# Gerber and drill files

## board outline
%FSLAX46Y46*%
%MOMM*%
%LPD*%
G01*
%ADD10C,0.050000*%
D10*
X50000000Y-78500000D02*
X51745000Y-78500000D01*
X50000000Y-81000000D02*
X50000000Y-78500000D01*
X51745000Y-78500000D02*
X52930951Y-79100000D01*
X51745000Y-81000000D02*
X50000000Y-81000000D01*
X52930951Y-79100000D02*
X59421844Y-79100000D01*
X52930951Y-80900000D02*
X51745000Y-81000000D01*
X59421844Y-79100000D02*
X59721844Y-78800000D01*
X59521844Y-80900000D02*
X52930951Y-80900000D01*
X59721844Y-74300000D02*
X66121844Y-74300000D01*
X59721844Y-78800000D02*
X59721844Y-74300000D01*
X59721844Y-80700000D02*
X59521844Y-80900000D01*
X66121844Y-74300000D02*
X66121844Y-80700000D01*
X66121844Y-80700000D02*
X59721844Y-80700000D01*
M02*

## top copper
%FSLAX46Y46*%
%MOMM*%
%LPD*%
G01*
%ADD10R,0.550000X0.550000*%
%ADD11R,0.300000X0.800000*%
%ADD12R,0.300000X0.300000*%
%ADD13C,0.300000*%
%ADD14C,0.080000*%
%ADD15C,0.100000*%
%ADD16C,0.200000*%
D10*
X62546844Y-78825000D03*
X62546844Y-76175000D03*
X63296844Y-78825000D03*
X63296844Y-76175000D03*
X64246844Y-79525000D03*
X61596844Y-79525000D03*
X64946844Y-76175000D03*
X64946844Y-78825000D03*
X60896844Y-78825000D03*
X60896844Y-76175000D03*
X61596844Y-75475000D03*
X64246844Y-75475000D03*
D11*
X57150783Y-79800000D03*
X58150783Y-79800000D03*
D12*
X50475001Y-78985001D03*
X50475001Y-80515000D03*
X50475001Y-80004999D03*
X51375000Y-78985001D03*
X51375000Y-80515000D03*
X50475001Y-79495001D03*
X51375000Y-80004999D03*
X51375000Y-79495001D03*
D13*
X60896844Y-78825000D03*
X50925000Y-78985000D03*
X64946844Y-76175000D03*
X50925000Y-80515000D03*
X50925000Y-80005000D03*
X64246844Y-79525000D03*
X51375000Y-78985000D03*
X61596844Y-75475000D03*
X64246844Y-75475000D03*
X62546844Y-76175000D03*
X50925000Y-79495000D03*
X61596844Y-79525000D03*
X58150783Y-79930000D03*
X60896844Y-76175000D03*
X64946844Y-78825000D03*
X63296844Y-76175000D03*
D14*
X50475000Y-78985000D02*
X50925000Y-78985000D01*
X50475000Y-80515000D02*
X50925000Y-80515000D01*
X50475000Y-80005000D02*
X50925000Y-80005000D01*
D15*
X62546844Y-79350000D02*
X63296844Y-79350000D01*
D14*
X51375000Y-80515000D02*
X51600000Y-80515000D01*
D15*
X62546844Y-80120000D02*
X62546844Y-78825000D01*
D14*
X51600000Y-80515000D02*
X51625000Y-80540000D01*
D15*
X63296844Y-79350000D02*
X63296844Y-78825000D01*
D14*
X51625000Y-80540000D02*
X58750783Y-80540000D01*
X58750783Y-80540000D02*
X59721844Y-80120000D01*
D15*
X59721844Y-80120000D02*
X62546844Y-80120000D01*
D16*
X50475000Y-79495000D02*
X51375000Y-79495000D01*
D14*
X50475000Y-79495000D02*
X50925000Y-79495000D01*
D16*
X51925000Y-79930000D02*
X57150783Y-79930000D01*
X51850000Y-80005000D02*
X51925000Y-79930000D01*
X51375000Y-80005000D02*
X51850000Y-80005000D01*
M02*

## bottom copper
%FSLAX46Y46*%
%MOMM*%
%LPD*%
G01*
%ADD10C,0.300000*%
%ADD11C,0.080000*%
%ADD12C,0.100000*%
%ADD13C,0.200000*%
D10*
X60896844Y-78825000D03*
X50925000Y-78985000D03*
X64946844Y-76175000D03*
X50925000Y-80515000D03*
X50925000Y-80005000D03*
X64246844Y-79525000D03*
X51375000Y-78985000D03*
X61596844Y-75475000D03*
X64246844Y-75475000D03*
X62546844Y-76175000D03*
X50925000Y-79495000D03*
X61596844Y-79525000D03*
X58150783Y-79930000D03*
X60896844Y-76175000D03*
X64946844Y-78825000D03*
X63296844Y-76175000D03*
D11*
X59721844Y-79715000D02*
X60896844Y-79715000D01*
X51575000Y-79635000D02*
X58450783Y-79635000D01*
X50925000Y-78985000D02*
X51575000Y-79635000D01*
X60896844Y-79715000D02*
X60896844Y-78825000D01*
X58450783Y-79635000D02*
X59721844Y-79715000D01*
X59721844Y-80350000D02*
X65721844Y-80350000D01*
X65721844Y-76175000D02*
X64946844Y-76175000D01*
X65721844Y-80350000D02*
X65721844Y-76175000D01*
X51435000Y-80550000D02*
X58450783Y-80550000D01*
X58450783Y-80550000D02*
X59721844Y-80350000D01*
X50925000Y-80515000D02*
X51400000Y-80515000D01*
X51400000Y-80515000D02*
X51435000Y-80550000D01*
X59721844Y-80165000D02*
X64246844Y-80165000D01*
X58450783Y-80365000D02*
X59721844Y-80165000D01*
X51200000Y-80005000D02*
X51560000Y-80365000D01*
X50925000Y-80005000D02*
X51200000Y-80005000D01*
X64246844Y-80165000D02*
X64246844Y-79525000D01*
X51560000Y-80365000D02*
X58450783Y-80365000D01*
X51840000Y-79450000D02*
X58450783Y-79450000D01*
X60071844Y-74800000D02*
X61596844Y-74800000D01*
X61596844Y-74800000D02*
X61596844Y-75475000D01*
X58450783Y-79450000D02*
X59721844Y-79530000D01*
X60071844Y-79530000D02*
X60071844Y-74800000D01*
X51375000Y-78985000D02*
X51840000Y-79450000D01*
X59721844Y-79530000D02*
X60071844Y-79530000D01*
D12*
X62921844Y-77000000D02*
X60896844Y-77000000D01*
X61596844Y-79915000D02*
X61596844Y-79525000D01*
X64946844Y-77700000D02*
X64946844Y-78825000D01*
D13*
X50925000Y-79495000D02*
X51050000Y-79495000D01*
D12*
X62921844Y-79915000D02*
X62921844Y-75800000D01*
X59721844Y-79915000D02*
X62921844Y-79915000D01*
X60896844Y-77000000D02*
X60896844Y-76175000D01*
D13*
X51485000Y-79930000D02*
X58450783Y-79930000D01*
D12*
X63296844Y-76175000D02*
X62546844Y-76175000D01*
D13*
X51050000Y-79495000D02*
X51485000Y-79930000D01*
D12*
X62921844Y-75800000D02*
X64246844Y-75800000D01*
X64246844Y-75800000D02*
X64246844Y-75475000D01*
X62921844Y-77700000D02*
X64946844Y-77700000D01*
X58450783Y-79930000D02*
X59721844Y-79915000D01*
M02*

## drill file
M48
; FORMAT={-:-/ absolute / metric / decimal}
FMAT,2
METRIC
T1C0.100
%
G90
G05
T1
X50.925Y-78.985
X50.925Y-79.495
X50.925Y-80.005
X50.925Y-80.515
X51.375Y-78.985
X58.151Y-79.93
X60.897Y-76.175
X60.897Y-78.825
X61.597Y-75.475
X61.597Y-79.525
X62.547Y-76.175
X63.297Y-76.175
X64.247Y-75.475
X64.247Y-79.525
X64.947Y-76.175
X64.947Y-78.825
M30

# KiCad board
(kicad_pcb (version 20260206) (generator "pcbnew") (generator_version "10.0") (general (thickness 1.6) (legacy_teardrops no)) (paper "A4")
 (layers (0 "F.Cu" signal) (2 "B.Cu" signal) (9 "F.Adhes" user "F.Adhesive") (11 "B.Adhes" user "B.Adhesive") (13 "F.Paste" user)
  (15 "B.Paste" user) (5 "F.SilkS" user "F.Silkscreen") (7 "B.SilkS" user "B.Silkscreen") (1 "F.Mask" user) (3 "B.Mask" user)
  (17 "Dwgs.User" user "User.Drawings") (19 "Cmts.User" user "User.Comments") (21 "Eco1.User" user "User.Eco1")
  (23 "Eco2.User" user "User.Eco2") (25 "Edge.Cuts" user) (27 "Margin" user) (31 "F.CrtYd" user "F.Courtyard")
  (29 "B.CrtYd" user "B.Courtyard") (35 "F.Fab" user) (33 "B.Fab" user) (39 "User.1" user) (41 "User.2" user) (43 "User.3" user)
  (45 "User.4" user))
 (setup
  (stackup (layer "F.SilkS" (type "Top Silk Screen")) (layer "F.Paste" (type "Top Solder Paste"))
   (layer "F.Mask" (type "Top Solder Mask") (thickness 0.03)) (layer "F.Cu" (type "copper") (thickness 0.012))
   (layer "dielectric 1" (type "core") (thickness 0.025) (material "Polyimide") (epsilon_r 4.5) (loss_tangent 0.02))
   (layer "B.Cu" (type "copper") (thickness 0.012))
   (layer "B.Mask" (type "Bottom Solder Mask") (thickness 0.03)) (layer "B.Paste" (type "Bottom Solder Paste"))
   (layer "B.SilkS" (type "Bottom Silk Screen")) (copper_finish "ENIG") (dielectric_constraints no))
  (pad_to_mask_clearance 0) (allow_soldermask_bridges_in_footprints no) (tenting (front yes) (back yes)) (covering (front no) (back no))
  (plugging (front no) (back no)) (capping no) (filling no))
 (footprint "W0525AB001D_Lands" (layer "F.Cu") (at 57.650783 79.93)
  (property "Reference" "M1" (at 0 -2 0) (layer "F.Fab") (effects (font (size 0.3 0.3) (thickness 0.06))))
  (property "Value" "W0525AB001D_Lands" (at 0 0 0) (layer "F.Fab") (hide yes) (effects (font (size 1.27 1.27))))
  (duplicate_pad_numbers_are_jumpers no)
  (pad "1" smd rect (at -0.5 -0.13) (size 0.3 0.8) (layers "F.Cu" "F.Mask") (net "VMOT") (solder_mask_margin 0.05) (thermal_bridge_angle 45))
  (pad "2" smd rect (at 0.5 -0.13) (size 0.3 0.8) (layers "F.Cu" "F.Mask") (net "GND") (solder_mask_margin 0.05) (thermal_bridge_angle 45)))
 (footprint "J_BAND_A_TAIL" (layer "F.Cu") (at 50.9 79.75)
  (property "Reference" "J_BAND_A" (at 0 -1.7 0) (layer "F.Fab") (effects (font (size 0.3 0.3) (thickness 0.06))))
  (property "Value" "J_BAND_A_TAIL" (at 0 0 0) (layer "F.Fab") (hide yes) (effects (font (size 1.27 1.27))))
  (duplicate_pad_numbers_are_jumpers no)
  (pad "1" smd rect (at -0.424999 -0.764999) (size 0.3 0.3) (layers "F.Cu" "F.Mask") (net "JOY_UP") (solder_mask_margin 0.05)
   (thermal_bridge_angle 45))
  (pad "2" smd rect (at -0.424999 0.765) (size 0.3 0.3) (layers "F.Cu" "F.Mask") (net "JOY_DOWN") (solder_mask_margin 0.05)
   (thermal_bridge_angle 45))
  (pad "3" smd rect (at -0.424999 0.254999) (size 0.3 0.3) (layers "F.Cu" "F.Mask") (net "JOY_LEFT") (solder_mask_margin 0.05)
   (thermal_bridge_angle 45))
  (pad "4" smd rect (at 0.475 -0.764999) (size 0.3 0.3) (layers "F.Cu" "F.Mask") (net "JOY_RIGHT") (solder_mask_margin 0.05)
   (thermal_bridge_angle 45))
  (pad "5" smd rect (at 0.475 0.765) (size 0.3 0.3) (layers "F.Cu" "F.Mask") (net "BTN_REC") (solder_mask_margin 0.05)
   (thermal_bridge_angle 45))
  (pad "6" smd rect (at -0.424999 -0.254999) (size 0.3 0.3) (layers "F.Cu" "F.Mask") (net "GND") (solder_mask_margin 0.05)
   (thermal_bridge_angle 45))
  (pad "7" smd rect (at 0.475 0.254999) (size 0.3 0.3) (layers "F.Cu" "F.Mask") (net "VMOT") (solder_mask_margin 0.05)
   (thermal_bridge_angle 45))
  (pad "8" smd rect (at 0.475 -0.254999) (size 0.3 0.3) (layers "F.Cu" "F.Mask") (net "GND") (solder_mask_margin 0.05)
   (thermal_bridge_angle 45)))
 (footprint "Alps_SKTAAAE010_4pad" (layer "F.Cu") (at 62.921844 77.5 90)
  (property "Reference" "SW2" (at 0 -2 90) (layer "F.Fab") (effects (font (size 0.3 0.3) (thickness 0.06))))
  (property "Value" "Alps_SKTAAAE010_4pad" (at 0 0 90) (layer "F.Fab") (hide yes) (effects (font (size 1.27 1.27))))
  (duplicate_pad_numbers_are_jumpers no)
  (pad "1" smd rect (at -1.325 -0.375 90) (size 0.55 0.55) (layers "F.Cu" "F.Mask") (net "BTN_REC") (solder_mask_margin 0.05)
   (thermal_bridge_angle 45))
  (pad "2" smd rect (at 1.325 -0.375 90) (size 0.55 0.55) (layers "F.Cu" "F.Mask" "F.Paste") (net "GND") (solder_mask_margin 0.05)
   (thermal_bridge_angle 45))
  (pad "3" smd rect (at -1.325 0.375 90) (size 0.55 0.55) (layers "F.Cu" "F.Mask" "F.Paste") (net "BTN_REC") (solder_mask_margin 0.05)
   (thermal_bridge_angle 45))
  (pad "4" smd rect (at 1.325 0.375 90) (size 0.55 0.55) (layers "F.Cu" "F.Mask" "F.Paste") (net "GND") (solder_mask_margin 0.05)
   (thermal_bridge_angle 45)))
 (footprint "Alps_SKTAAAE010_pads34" (layer "F.Cu") (at 62.921844 75.1)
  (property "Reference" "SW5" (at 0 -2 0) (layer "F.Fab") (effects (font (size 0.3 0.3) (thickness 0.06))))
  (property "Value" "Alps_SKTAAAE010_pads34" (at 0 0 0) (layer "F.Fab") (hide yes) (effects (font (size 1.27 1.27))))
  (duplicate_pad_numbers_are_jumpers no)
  (pad "3" smd rect (at -1.325 0.375) (size 0.55 0.55) (layers "F.Cu" "F.Mask" "F.Paste") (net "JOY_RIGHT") (solder_mask_margin 0.05)
   (thermal_bridge_angle 45))
  (pad "4" smd rect (at 1.325 0.375) (size 0.55 0.55) (layers "F.Cu" "F.Mask" "F.Paste") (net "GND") (solder_mask_margin 0.05)
   (thermal_bridge_angle 45)))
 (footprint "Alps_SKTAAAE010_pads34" (layer "F.Cu") (at 65.321844 77.5 -90)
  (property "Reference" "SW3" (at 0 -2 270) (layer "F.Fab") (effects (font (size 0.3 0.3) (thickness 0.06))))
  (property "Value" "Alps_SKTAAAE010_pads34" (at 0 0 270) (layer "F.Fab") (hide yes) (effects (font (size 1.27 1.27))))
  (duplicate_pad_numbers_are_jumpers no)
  (pad "3" smd rect (at -1.325 0.375 270) (size 0.55 0.55) (layers "F.Cu" "F.Mask" "F.Paste") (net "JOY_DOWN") (solder_mask_margin 0.05)
   (thermal_bridge_angle 45))
  (pad "4" smd rect (at 1.325 0.375 270) (size 0.55 0.55) (layers "F.Cu" "F.Mask" "F.Paste") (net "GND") (solder_mask_margin 0.05)
   (thermal_bridge_angle 45)))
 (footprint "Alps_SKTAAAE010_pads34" (layer "F.Cu") (at 62.921844 79.9 180)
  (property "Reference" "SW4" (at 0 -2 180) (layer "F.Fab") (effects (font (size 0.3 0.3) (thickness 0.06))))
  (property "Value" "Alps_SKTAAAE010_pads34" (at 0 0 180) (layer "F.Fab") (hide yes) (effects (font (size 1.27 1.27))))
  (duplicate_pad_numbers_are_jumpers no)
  (pad "3" smd rect (at -1.325 0.375 180) (size 0.55 0.55) (layers "F.Cu" "F.Mask" "F.Paste") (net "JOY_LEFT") (solder_mask_margin 0.05)
   (thermal_bridge_angle 45))
  (pad "4" smd rect (at 1.325 0.375 180) (size 0.55 0.55) (layers "F.Cu" "F.Mask" "F.Paste") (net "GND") (solder_mask_margin 0.05)
   (thermal_bridge_angle 45)))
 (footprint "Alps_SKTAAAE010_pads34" (layer "F.Cu") (at 60.521844 77.5 90)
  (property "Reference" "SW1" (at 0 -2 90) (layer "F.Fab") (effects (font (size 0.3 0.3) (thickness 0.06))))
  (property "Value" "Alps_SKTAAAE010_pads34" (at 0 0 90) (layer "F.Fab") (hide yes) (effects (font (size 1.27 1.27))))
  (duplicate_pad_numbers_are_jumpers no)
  (pad "3" smd rect (at -1.325 0.375 90) (size 0.55 0.55) (layers "F.Cu" "F.Mask" "F.Paste") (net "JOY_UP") (solder_mask_margin 0.05)
   (thermal_bridge_angle 45))
  (pad "4" smd rect (at 1.325 0.375 90) (size 0.55 0.55) (layers "F.Cu" "F.Mask" "F.Paste") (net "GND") (solder_mask_margin 0.05)
   (thermal_bridge_angle 45)))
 (gr_line (start 50 78.5) (end 51.745 78.5) (stroke (width 0.05) (type default)) (layer "Edge.Cuts"))
 (gr_line (start 50 81) (end 50 78.5) (stroke (width 0.05) (type default)) (layer "Edge.Cuts"))
 (gr_line (start 51.745 78.5) (end 52.930951 79.1) (stroke (width 0.05) (type default)) (layer "Edge.Cuts"))
 (gr_line (start 51.745 81) (end 50 81) (stroke (width 0.05) (type default)) (layer "Edge.Cuts"))
 (gr_line (start 52.930951 79.1) (end 59.421844 79.1) (stroke (width 0.05) (type default)) (layer "Edge.Cuts"))
 (gr_line (start 52.930951 80.9) (end 51.745 81) (stroke (width 0.05) (type default)) (layer "Edge.Cuts"))
 (gr_line (start 59.421844 79.1) (end 59.721844 78.8) (stroke (width 0.05) (type default)) (layer "Edge.Cuts"))
 (gr_line (start 59.521844 80.9) (end 52.930951 80.9) (stroke (width 0.05) (type default)) (layer "Edge.Cuts"))
 (gr_line (start 59.721844 74.3) (end 66.121844 74.3) (stroke (width 0.05) (type default)) (layer "Edge.Cuts"))
 (gr_line (start 59.721844 78.8) (end 59.721844 74.3) (stroke (width 0.05) (type default)) (layer "Edge.Cuts"))
 (gr_line (start 59.721844 80.7) (end 59.521844 80.9) (stroke (width 0.05) (type default)) (layer "Edge.Cuts"))
 (gr_line (start 66.121844 74.3) (end 66.121844 80.7) (stroke (width 0.05) (type default)) (layer "Edge.Cuts"))
 (gr_line (start 66.121844 80.7) (end 59.721844 80.7) (stroke (width 0.05) (type default)) (layer "Edge.Cuts"))
 (segment (start 51.925 79.93) (end 57.150783 79.93) (width 0.2) (layer "F.Cu") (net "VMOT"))
 (segment (start 51.85 80.005) (end 51.925 79.93) (width 0.2) (layer "F.Cu") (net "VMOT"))
 (segment (start 51.375 80.005) (end 51.85 80.005) (width 0.2) (layer "F.Cu") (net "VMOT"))
 (segment (start 50.475 79.495) (end 50.925 79.495) (width 0.08) (layer "F.Cu") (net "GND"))
 (segment (start 50.475 79.495) (end 51.375 79.495) (width 0.2) (layer "F.Cu") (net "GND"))
 (via (at 63.296844 76.175) (size 0.3) (drill 0.1) (layers "F.Cu" "B.Cu") (tenting (front yes) (back yes)) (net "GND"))
 (via (at 62.546844 76.175) (size 0.3) (drill 0.1) (layers "F.Cu" "B.Cu") (tenting (front yes) (back yes)) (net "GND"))
 (via (at 58.150783 79.93) (size 0.3) (drill 0.1) (layers "F.Cu" "B.Cu") (tenting (front yes) (back yes)) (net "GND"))
 (via (at 60.896844 76.175) (size 0.3) (drill 0.1) (layers "F.Cu" "B.Cu") (tenting (front yes) (back yes)) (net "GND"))
 (via (at 64.946844 78.825) (size 0.3) (drill 0.1) (layers "F.Cu" "B.Cu") (tenting (front yes) (back yes)) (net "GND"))
 (via (at 64.246844 75.475) (size 0.3) (drill 0.1) (layers "F.Cu" "B.Cu") (tenting (front yes) (back yes)) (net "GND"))
 (via (at 50.925 79.495) (size 0.3) (drill 0.1) (layers "F.Cu" "B.Cu") (tenting (front yes) (back yes)) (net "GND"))
 (via (at 61.596844 79.525) (size 0.3) (drill 0.1) (layers "F.Cu" "B.Cu") (tenting (front yes) (back yes)) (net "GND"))
 (segment (start 64.946844 77.7) (end 64.946844 78.825) (width 0.1) (layer "B.Cu") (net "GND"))
 (segment (start 64.246844 75.8) (end 64.246844 75.475) (width 0.1) (layer "B.Cu") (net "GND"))
 (segment (start 51.485 79.93) (end 58.450783 79.93) (width 0.2) (layer "B.Cu") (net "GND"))
 (segment (start 58.450783 79.93) (end 59.721844 79.915) (width 0.1) (layer "B.Cu") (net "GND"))
 (segment (start 59.721844 79.915) (end 62.921844 79.915) (width 0.1) (layer "B.Cu") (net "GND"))
 (segment (start 62.921844 75.8) (end 64.246844 75.8) (width 0.1) (layer "B.Cu") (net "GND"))
 (segment (start 50.925 79.495) (end 51.05 79.495) (width 0.2) (layer "B.Cu") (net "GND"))
 (segment (start 51.05 79.495) (end 51.485 79.93) (width 0.2) (layer "B.Cu") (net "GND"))
 (segment (start 62.921844 77.7) (end 64.946844 77.7) (width 0.1) (layer "B.Cu") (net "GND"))
 (segment (start 61.596844 79.915) (end 61.596844 79.525) (width 0.1) (layer "B.Cu") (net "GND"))
 (segment (start 63.296844 76.175) (end 62.546844 76.175) (width 0.1) (layer "B.Cu") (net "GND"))
 (segment (start 60.896844 77) (end 60.896844 76.175) (width 0.1) (layer "B.Cu") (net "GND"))
 (segment (start 62.921844 77) (end 60.896844 77) (width 0.1) (layer "B.Cu") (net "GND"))
 (segment (start 62.921844 79.915) (end 62.921844 75.8) (width 0.1) (layer "B.Cu") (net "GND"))
 (segment (start 50.475 78.985) (end 50.925 78.985) (width 0.08) (layer "F.Cu") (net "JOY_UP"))
 (via (at 60.896844 78.825) (size 0.3) (drill 0.1) (layers "F.Cu" "B.Cu") (tenting (front yes) (back yes)) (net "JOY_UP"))
 (via (at 50.925 78.985) (size 0.3) (drill 0.1) (layers "F.Cu" "B.Cu") (tenting (front yes) (back yes)) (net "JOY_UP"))
 (segment (start 51.575 79.635) (end 58.450783 79.635) (width 0.08) (layer "B.Cu") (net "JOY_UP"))
 (segment (start 60.896844 79.715) (end 60.896844 78.825) (width 0.08) (layer "B.Cu") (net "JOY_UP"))
 (segment (start 59.721844 79.715) (end 60.896844 79.715) (width 0.08) (layer "B.Cu") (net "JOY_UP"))
 (segment (start 50.925 78.985) (end 51.575 79.635) (width 0.08) (layer "B.Cu") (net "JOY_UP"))
 (segment (start 58.450783 79.635) (end 59.721844 79.715) (width 0.08) (layer "B.Cu") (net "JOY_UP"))
 (segment (start 50.475 80.515) (end 50.925 80.515) (width 0.08) (layer "F.Cu") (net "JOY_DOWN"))
 (via (at 50.925 80.515) (size 0.3) (drill 0.1) (layers "F.Cu" "B.Cu") (tenting (front yes) (back yes)) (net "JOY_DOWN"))
 (via (at 64.946844 76.175) (size 0.3) (drill 0.1) (layers "F.Cu" "B.Cu") (tenting (front yes) (back yes)) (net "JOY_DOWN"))
 (segment (start 59.721844 80.35) (end 65.721844 80.35) (width 0.08) (layer "B.Cu") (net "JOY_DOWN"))
 (segment (start 65.721844 80.35) (end 65.721844 76.175) (width 0.08) (layer "B.Cu") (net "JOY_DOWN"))
 (segment (start 51.4 80.515) (end 51.435 80.55) (width 0.08) (layer "B.Cu") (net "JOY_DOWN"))
 (segment (start 65.721844 76.175) (end 64.946844 76.175) (width 0.08) (layer "B.Cu") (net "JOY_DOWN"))
 (segment (start 50.925 80.515) (end 51.4 80.515) (width 0.08) (layer "B.Cu") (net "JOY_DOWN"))
 (segment (start 58.450783 80.55) (end 59.721844 80.35) (width 0.08) (layer "B.Cu") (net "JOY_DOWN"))
 (segment (start 51.435 80.55) (end 58.450783 80.55) (width 0.08) (layer "B.Cu") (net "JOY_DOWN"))
 (segment (start 50.475 80.005) (end 50.925 80.005) (width 0.08) (layer "F.Cu") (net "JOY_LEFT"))
 (via (at 50.925 80.005) (size 0.3) (drill 0.1) (layers "F.Cu" "B.Cu") (tenting (front yes) (back yes)) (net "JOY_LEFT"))
 (via (at 64.246844 79.525) (size 0.3) (drill 0.1) (layers "F.Cu" "B.Cu") (tenting (front yes) (back yes)) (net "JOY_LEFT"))
 (segment (start 51.2 80.005) (end 51.56 80.365) (width 0.08) (layer "B.Cu") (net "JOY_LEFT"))
 (segment (start 51.56 80.365) (end 58.450783 80.365) (width 0.08) (layer "B.Cu") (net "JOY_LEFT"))
 (segment (start 59.721844 80.165) (end 64.246844 80.165) (width 0.08) (layer "B.Cu") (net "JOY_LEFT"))
 (segment (start 50.925 80.005) (end 51.2 80.005) (width 0.08) (layer "B.Cu") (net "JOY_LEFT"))
 (segment (start 58.450783 80.365) (end 59.721844 80.165) (width 0.08) (layer "B.Cu") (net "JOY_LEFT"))
 (segment (start 64.246844 80.165) (end 64.246844 79.525) (width 0.08) (layer "B.Cu") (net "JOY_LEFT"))
 (via (at 61.596844 75.475) (size 0.3) (drill 0.1) (layers "F.Cu" "B.Cu") (tenting (front yes) (back yes)) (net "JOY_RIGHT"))
 (via (at 51.375 78.985) (size 0.3) (drill 0.1) (layers "F.Cu" "B.Cu") (tenting (front yes) (back yes)) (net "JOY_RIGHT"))
 (segment (start 60.071844 79.53) (end 60.071844 74.8) (width 0.08) (layer "B.Cu") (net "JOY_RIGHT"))
 (segment (start 58.450783 79.45) (end 59.721844 79.53) (width 0.08) (layer "B.Cu") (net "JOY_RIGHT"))
 (segment (start 59.721844 79.53) (end 60.071844 79.53) (width 0.08) (layer "B.Cu") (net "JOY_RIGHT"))
 (segment (start 51.84 79.45) (end 58.450783 79.45) (width 0.08) (layer "B.Cu") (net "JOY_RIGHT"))
 (segment (start 60.071844 74.8) (end 61.596844 74.8) (width 0.08) (layer "B.Cu") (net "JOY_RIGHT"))
 (segment (start 61.596844 74.8) (end 61.596844 75.475) (width 0.08) (layer "B.Cu") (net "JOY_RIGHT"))
 (segment (start 51.375 78.985) (end 51.84 79.45) (width 0.08) (layer "B.Cu") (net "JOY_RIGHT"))
 (segment (start 62.546844 79.35) (end 63.296844 79.35) (width 0.1) (layer "F.Cu") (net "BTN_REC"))
 (segment (start 62.546844 80.12) (end 62.546844 78.825) (width 0.1) (layer "F.Cu") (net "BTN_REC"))
 (segment (start 51.625 80.54) (end 58.750783 80.54) (width 0.08) (layer "F.Cu") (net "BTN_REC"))
 (segment (start 59.721844 80.12) (end 62.546844 80.12) (width 0.1) (layer "F.Cu") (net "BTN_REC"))
 (segment (start 58.750783 80.54) (end 59.721844 80.12) (width 0.08) (layer "F.Cu") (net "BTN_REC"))
 (segment (start 51.6 80.515) (end 51.625 80.54) (width 0.08) (layer "F.Cu") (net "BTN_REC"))
 (segment (start 63.296844 79.35) (end 63.296844 78.825) (width 0.1) (layer "F.Cu") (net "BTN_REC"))
 (segment (start 51.375 80.515) (end 51.6 80.515) (width 0.08) (layer "F.Cu") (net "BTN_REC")))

